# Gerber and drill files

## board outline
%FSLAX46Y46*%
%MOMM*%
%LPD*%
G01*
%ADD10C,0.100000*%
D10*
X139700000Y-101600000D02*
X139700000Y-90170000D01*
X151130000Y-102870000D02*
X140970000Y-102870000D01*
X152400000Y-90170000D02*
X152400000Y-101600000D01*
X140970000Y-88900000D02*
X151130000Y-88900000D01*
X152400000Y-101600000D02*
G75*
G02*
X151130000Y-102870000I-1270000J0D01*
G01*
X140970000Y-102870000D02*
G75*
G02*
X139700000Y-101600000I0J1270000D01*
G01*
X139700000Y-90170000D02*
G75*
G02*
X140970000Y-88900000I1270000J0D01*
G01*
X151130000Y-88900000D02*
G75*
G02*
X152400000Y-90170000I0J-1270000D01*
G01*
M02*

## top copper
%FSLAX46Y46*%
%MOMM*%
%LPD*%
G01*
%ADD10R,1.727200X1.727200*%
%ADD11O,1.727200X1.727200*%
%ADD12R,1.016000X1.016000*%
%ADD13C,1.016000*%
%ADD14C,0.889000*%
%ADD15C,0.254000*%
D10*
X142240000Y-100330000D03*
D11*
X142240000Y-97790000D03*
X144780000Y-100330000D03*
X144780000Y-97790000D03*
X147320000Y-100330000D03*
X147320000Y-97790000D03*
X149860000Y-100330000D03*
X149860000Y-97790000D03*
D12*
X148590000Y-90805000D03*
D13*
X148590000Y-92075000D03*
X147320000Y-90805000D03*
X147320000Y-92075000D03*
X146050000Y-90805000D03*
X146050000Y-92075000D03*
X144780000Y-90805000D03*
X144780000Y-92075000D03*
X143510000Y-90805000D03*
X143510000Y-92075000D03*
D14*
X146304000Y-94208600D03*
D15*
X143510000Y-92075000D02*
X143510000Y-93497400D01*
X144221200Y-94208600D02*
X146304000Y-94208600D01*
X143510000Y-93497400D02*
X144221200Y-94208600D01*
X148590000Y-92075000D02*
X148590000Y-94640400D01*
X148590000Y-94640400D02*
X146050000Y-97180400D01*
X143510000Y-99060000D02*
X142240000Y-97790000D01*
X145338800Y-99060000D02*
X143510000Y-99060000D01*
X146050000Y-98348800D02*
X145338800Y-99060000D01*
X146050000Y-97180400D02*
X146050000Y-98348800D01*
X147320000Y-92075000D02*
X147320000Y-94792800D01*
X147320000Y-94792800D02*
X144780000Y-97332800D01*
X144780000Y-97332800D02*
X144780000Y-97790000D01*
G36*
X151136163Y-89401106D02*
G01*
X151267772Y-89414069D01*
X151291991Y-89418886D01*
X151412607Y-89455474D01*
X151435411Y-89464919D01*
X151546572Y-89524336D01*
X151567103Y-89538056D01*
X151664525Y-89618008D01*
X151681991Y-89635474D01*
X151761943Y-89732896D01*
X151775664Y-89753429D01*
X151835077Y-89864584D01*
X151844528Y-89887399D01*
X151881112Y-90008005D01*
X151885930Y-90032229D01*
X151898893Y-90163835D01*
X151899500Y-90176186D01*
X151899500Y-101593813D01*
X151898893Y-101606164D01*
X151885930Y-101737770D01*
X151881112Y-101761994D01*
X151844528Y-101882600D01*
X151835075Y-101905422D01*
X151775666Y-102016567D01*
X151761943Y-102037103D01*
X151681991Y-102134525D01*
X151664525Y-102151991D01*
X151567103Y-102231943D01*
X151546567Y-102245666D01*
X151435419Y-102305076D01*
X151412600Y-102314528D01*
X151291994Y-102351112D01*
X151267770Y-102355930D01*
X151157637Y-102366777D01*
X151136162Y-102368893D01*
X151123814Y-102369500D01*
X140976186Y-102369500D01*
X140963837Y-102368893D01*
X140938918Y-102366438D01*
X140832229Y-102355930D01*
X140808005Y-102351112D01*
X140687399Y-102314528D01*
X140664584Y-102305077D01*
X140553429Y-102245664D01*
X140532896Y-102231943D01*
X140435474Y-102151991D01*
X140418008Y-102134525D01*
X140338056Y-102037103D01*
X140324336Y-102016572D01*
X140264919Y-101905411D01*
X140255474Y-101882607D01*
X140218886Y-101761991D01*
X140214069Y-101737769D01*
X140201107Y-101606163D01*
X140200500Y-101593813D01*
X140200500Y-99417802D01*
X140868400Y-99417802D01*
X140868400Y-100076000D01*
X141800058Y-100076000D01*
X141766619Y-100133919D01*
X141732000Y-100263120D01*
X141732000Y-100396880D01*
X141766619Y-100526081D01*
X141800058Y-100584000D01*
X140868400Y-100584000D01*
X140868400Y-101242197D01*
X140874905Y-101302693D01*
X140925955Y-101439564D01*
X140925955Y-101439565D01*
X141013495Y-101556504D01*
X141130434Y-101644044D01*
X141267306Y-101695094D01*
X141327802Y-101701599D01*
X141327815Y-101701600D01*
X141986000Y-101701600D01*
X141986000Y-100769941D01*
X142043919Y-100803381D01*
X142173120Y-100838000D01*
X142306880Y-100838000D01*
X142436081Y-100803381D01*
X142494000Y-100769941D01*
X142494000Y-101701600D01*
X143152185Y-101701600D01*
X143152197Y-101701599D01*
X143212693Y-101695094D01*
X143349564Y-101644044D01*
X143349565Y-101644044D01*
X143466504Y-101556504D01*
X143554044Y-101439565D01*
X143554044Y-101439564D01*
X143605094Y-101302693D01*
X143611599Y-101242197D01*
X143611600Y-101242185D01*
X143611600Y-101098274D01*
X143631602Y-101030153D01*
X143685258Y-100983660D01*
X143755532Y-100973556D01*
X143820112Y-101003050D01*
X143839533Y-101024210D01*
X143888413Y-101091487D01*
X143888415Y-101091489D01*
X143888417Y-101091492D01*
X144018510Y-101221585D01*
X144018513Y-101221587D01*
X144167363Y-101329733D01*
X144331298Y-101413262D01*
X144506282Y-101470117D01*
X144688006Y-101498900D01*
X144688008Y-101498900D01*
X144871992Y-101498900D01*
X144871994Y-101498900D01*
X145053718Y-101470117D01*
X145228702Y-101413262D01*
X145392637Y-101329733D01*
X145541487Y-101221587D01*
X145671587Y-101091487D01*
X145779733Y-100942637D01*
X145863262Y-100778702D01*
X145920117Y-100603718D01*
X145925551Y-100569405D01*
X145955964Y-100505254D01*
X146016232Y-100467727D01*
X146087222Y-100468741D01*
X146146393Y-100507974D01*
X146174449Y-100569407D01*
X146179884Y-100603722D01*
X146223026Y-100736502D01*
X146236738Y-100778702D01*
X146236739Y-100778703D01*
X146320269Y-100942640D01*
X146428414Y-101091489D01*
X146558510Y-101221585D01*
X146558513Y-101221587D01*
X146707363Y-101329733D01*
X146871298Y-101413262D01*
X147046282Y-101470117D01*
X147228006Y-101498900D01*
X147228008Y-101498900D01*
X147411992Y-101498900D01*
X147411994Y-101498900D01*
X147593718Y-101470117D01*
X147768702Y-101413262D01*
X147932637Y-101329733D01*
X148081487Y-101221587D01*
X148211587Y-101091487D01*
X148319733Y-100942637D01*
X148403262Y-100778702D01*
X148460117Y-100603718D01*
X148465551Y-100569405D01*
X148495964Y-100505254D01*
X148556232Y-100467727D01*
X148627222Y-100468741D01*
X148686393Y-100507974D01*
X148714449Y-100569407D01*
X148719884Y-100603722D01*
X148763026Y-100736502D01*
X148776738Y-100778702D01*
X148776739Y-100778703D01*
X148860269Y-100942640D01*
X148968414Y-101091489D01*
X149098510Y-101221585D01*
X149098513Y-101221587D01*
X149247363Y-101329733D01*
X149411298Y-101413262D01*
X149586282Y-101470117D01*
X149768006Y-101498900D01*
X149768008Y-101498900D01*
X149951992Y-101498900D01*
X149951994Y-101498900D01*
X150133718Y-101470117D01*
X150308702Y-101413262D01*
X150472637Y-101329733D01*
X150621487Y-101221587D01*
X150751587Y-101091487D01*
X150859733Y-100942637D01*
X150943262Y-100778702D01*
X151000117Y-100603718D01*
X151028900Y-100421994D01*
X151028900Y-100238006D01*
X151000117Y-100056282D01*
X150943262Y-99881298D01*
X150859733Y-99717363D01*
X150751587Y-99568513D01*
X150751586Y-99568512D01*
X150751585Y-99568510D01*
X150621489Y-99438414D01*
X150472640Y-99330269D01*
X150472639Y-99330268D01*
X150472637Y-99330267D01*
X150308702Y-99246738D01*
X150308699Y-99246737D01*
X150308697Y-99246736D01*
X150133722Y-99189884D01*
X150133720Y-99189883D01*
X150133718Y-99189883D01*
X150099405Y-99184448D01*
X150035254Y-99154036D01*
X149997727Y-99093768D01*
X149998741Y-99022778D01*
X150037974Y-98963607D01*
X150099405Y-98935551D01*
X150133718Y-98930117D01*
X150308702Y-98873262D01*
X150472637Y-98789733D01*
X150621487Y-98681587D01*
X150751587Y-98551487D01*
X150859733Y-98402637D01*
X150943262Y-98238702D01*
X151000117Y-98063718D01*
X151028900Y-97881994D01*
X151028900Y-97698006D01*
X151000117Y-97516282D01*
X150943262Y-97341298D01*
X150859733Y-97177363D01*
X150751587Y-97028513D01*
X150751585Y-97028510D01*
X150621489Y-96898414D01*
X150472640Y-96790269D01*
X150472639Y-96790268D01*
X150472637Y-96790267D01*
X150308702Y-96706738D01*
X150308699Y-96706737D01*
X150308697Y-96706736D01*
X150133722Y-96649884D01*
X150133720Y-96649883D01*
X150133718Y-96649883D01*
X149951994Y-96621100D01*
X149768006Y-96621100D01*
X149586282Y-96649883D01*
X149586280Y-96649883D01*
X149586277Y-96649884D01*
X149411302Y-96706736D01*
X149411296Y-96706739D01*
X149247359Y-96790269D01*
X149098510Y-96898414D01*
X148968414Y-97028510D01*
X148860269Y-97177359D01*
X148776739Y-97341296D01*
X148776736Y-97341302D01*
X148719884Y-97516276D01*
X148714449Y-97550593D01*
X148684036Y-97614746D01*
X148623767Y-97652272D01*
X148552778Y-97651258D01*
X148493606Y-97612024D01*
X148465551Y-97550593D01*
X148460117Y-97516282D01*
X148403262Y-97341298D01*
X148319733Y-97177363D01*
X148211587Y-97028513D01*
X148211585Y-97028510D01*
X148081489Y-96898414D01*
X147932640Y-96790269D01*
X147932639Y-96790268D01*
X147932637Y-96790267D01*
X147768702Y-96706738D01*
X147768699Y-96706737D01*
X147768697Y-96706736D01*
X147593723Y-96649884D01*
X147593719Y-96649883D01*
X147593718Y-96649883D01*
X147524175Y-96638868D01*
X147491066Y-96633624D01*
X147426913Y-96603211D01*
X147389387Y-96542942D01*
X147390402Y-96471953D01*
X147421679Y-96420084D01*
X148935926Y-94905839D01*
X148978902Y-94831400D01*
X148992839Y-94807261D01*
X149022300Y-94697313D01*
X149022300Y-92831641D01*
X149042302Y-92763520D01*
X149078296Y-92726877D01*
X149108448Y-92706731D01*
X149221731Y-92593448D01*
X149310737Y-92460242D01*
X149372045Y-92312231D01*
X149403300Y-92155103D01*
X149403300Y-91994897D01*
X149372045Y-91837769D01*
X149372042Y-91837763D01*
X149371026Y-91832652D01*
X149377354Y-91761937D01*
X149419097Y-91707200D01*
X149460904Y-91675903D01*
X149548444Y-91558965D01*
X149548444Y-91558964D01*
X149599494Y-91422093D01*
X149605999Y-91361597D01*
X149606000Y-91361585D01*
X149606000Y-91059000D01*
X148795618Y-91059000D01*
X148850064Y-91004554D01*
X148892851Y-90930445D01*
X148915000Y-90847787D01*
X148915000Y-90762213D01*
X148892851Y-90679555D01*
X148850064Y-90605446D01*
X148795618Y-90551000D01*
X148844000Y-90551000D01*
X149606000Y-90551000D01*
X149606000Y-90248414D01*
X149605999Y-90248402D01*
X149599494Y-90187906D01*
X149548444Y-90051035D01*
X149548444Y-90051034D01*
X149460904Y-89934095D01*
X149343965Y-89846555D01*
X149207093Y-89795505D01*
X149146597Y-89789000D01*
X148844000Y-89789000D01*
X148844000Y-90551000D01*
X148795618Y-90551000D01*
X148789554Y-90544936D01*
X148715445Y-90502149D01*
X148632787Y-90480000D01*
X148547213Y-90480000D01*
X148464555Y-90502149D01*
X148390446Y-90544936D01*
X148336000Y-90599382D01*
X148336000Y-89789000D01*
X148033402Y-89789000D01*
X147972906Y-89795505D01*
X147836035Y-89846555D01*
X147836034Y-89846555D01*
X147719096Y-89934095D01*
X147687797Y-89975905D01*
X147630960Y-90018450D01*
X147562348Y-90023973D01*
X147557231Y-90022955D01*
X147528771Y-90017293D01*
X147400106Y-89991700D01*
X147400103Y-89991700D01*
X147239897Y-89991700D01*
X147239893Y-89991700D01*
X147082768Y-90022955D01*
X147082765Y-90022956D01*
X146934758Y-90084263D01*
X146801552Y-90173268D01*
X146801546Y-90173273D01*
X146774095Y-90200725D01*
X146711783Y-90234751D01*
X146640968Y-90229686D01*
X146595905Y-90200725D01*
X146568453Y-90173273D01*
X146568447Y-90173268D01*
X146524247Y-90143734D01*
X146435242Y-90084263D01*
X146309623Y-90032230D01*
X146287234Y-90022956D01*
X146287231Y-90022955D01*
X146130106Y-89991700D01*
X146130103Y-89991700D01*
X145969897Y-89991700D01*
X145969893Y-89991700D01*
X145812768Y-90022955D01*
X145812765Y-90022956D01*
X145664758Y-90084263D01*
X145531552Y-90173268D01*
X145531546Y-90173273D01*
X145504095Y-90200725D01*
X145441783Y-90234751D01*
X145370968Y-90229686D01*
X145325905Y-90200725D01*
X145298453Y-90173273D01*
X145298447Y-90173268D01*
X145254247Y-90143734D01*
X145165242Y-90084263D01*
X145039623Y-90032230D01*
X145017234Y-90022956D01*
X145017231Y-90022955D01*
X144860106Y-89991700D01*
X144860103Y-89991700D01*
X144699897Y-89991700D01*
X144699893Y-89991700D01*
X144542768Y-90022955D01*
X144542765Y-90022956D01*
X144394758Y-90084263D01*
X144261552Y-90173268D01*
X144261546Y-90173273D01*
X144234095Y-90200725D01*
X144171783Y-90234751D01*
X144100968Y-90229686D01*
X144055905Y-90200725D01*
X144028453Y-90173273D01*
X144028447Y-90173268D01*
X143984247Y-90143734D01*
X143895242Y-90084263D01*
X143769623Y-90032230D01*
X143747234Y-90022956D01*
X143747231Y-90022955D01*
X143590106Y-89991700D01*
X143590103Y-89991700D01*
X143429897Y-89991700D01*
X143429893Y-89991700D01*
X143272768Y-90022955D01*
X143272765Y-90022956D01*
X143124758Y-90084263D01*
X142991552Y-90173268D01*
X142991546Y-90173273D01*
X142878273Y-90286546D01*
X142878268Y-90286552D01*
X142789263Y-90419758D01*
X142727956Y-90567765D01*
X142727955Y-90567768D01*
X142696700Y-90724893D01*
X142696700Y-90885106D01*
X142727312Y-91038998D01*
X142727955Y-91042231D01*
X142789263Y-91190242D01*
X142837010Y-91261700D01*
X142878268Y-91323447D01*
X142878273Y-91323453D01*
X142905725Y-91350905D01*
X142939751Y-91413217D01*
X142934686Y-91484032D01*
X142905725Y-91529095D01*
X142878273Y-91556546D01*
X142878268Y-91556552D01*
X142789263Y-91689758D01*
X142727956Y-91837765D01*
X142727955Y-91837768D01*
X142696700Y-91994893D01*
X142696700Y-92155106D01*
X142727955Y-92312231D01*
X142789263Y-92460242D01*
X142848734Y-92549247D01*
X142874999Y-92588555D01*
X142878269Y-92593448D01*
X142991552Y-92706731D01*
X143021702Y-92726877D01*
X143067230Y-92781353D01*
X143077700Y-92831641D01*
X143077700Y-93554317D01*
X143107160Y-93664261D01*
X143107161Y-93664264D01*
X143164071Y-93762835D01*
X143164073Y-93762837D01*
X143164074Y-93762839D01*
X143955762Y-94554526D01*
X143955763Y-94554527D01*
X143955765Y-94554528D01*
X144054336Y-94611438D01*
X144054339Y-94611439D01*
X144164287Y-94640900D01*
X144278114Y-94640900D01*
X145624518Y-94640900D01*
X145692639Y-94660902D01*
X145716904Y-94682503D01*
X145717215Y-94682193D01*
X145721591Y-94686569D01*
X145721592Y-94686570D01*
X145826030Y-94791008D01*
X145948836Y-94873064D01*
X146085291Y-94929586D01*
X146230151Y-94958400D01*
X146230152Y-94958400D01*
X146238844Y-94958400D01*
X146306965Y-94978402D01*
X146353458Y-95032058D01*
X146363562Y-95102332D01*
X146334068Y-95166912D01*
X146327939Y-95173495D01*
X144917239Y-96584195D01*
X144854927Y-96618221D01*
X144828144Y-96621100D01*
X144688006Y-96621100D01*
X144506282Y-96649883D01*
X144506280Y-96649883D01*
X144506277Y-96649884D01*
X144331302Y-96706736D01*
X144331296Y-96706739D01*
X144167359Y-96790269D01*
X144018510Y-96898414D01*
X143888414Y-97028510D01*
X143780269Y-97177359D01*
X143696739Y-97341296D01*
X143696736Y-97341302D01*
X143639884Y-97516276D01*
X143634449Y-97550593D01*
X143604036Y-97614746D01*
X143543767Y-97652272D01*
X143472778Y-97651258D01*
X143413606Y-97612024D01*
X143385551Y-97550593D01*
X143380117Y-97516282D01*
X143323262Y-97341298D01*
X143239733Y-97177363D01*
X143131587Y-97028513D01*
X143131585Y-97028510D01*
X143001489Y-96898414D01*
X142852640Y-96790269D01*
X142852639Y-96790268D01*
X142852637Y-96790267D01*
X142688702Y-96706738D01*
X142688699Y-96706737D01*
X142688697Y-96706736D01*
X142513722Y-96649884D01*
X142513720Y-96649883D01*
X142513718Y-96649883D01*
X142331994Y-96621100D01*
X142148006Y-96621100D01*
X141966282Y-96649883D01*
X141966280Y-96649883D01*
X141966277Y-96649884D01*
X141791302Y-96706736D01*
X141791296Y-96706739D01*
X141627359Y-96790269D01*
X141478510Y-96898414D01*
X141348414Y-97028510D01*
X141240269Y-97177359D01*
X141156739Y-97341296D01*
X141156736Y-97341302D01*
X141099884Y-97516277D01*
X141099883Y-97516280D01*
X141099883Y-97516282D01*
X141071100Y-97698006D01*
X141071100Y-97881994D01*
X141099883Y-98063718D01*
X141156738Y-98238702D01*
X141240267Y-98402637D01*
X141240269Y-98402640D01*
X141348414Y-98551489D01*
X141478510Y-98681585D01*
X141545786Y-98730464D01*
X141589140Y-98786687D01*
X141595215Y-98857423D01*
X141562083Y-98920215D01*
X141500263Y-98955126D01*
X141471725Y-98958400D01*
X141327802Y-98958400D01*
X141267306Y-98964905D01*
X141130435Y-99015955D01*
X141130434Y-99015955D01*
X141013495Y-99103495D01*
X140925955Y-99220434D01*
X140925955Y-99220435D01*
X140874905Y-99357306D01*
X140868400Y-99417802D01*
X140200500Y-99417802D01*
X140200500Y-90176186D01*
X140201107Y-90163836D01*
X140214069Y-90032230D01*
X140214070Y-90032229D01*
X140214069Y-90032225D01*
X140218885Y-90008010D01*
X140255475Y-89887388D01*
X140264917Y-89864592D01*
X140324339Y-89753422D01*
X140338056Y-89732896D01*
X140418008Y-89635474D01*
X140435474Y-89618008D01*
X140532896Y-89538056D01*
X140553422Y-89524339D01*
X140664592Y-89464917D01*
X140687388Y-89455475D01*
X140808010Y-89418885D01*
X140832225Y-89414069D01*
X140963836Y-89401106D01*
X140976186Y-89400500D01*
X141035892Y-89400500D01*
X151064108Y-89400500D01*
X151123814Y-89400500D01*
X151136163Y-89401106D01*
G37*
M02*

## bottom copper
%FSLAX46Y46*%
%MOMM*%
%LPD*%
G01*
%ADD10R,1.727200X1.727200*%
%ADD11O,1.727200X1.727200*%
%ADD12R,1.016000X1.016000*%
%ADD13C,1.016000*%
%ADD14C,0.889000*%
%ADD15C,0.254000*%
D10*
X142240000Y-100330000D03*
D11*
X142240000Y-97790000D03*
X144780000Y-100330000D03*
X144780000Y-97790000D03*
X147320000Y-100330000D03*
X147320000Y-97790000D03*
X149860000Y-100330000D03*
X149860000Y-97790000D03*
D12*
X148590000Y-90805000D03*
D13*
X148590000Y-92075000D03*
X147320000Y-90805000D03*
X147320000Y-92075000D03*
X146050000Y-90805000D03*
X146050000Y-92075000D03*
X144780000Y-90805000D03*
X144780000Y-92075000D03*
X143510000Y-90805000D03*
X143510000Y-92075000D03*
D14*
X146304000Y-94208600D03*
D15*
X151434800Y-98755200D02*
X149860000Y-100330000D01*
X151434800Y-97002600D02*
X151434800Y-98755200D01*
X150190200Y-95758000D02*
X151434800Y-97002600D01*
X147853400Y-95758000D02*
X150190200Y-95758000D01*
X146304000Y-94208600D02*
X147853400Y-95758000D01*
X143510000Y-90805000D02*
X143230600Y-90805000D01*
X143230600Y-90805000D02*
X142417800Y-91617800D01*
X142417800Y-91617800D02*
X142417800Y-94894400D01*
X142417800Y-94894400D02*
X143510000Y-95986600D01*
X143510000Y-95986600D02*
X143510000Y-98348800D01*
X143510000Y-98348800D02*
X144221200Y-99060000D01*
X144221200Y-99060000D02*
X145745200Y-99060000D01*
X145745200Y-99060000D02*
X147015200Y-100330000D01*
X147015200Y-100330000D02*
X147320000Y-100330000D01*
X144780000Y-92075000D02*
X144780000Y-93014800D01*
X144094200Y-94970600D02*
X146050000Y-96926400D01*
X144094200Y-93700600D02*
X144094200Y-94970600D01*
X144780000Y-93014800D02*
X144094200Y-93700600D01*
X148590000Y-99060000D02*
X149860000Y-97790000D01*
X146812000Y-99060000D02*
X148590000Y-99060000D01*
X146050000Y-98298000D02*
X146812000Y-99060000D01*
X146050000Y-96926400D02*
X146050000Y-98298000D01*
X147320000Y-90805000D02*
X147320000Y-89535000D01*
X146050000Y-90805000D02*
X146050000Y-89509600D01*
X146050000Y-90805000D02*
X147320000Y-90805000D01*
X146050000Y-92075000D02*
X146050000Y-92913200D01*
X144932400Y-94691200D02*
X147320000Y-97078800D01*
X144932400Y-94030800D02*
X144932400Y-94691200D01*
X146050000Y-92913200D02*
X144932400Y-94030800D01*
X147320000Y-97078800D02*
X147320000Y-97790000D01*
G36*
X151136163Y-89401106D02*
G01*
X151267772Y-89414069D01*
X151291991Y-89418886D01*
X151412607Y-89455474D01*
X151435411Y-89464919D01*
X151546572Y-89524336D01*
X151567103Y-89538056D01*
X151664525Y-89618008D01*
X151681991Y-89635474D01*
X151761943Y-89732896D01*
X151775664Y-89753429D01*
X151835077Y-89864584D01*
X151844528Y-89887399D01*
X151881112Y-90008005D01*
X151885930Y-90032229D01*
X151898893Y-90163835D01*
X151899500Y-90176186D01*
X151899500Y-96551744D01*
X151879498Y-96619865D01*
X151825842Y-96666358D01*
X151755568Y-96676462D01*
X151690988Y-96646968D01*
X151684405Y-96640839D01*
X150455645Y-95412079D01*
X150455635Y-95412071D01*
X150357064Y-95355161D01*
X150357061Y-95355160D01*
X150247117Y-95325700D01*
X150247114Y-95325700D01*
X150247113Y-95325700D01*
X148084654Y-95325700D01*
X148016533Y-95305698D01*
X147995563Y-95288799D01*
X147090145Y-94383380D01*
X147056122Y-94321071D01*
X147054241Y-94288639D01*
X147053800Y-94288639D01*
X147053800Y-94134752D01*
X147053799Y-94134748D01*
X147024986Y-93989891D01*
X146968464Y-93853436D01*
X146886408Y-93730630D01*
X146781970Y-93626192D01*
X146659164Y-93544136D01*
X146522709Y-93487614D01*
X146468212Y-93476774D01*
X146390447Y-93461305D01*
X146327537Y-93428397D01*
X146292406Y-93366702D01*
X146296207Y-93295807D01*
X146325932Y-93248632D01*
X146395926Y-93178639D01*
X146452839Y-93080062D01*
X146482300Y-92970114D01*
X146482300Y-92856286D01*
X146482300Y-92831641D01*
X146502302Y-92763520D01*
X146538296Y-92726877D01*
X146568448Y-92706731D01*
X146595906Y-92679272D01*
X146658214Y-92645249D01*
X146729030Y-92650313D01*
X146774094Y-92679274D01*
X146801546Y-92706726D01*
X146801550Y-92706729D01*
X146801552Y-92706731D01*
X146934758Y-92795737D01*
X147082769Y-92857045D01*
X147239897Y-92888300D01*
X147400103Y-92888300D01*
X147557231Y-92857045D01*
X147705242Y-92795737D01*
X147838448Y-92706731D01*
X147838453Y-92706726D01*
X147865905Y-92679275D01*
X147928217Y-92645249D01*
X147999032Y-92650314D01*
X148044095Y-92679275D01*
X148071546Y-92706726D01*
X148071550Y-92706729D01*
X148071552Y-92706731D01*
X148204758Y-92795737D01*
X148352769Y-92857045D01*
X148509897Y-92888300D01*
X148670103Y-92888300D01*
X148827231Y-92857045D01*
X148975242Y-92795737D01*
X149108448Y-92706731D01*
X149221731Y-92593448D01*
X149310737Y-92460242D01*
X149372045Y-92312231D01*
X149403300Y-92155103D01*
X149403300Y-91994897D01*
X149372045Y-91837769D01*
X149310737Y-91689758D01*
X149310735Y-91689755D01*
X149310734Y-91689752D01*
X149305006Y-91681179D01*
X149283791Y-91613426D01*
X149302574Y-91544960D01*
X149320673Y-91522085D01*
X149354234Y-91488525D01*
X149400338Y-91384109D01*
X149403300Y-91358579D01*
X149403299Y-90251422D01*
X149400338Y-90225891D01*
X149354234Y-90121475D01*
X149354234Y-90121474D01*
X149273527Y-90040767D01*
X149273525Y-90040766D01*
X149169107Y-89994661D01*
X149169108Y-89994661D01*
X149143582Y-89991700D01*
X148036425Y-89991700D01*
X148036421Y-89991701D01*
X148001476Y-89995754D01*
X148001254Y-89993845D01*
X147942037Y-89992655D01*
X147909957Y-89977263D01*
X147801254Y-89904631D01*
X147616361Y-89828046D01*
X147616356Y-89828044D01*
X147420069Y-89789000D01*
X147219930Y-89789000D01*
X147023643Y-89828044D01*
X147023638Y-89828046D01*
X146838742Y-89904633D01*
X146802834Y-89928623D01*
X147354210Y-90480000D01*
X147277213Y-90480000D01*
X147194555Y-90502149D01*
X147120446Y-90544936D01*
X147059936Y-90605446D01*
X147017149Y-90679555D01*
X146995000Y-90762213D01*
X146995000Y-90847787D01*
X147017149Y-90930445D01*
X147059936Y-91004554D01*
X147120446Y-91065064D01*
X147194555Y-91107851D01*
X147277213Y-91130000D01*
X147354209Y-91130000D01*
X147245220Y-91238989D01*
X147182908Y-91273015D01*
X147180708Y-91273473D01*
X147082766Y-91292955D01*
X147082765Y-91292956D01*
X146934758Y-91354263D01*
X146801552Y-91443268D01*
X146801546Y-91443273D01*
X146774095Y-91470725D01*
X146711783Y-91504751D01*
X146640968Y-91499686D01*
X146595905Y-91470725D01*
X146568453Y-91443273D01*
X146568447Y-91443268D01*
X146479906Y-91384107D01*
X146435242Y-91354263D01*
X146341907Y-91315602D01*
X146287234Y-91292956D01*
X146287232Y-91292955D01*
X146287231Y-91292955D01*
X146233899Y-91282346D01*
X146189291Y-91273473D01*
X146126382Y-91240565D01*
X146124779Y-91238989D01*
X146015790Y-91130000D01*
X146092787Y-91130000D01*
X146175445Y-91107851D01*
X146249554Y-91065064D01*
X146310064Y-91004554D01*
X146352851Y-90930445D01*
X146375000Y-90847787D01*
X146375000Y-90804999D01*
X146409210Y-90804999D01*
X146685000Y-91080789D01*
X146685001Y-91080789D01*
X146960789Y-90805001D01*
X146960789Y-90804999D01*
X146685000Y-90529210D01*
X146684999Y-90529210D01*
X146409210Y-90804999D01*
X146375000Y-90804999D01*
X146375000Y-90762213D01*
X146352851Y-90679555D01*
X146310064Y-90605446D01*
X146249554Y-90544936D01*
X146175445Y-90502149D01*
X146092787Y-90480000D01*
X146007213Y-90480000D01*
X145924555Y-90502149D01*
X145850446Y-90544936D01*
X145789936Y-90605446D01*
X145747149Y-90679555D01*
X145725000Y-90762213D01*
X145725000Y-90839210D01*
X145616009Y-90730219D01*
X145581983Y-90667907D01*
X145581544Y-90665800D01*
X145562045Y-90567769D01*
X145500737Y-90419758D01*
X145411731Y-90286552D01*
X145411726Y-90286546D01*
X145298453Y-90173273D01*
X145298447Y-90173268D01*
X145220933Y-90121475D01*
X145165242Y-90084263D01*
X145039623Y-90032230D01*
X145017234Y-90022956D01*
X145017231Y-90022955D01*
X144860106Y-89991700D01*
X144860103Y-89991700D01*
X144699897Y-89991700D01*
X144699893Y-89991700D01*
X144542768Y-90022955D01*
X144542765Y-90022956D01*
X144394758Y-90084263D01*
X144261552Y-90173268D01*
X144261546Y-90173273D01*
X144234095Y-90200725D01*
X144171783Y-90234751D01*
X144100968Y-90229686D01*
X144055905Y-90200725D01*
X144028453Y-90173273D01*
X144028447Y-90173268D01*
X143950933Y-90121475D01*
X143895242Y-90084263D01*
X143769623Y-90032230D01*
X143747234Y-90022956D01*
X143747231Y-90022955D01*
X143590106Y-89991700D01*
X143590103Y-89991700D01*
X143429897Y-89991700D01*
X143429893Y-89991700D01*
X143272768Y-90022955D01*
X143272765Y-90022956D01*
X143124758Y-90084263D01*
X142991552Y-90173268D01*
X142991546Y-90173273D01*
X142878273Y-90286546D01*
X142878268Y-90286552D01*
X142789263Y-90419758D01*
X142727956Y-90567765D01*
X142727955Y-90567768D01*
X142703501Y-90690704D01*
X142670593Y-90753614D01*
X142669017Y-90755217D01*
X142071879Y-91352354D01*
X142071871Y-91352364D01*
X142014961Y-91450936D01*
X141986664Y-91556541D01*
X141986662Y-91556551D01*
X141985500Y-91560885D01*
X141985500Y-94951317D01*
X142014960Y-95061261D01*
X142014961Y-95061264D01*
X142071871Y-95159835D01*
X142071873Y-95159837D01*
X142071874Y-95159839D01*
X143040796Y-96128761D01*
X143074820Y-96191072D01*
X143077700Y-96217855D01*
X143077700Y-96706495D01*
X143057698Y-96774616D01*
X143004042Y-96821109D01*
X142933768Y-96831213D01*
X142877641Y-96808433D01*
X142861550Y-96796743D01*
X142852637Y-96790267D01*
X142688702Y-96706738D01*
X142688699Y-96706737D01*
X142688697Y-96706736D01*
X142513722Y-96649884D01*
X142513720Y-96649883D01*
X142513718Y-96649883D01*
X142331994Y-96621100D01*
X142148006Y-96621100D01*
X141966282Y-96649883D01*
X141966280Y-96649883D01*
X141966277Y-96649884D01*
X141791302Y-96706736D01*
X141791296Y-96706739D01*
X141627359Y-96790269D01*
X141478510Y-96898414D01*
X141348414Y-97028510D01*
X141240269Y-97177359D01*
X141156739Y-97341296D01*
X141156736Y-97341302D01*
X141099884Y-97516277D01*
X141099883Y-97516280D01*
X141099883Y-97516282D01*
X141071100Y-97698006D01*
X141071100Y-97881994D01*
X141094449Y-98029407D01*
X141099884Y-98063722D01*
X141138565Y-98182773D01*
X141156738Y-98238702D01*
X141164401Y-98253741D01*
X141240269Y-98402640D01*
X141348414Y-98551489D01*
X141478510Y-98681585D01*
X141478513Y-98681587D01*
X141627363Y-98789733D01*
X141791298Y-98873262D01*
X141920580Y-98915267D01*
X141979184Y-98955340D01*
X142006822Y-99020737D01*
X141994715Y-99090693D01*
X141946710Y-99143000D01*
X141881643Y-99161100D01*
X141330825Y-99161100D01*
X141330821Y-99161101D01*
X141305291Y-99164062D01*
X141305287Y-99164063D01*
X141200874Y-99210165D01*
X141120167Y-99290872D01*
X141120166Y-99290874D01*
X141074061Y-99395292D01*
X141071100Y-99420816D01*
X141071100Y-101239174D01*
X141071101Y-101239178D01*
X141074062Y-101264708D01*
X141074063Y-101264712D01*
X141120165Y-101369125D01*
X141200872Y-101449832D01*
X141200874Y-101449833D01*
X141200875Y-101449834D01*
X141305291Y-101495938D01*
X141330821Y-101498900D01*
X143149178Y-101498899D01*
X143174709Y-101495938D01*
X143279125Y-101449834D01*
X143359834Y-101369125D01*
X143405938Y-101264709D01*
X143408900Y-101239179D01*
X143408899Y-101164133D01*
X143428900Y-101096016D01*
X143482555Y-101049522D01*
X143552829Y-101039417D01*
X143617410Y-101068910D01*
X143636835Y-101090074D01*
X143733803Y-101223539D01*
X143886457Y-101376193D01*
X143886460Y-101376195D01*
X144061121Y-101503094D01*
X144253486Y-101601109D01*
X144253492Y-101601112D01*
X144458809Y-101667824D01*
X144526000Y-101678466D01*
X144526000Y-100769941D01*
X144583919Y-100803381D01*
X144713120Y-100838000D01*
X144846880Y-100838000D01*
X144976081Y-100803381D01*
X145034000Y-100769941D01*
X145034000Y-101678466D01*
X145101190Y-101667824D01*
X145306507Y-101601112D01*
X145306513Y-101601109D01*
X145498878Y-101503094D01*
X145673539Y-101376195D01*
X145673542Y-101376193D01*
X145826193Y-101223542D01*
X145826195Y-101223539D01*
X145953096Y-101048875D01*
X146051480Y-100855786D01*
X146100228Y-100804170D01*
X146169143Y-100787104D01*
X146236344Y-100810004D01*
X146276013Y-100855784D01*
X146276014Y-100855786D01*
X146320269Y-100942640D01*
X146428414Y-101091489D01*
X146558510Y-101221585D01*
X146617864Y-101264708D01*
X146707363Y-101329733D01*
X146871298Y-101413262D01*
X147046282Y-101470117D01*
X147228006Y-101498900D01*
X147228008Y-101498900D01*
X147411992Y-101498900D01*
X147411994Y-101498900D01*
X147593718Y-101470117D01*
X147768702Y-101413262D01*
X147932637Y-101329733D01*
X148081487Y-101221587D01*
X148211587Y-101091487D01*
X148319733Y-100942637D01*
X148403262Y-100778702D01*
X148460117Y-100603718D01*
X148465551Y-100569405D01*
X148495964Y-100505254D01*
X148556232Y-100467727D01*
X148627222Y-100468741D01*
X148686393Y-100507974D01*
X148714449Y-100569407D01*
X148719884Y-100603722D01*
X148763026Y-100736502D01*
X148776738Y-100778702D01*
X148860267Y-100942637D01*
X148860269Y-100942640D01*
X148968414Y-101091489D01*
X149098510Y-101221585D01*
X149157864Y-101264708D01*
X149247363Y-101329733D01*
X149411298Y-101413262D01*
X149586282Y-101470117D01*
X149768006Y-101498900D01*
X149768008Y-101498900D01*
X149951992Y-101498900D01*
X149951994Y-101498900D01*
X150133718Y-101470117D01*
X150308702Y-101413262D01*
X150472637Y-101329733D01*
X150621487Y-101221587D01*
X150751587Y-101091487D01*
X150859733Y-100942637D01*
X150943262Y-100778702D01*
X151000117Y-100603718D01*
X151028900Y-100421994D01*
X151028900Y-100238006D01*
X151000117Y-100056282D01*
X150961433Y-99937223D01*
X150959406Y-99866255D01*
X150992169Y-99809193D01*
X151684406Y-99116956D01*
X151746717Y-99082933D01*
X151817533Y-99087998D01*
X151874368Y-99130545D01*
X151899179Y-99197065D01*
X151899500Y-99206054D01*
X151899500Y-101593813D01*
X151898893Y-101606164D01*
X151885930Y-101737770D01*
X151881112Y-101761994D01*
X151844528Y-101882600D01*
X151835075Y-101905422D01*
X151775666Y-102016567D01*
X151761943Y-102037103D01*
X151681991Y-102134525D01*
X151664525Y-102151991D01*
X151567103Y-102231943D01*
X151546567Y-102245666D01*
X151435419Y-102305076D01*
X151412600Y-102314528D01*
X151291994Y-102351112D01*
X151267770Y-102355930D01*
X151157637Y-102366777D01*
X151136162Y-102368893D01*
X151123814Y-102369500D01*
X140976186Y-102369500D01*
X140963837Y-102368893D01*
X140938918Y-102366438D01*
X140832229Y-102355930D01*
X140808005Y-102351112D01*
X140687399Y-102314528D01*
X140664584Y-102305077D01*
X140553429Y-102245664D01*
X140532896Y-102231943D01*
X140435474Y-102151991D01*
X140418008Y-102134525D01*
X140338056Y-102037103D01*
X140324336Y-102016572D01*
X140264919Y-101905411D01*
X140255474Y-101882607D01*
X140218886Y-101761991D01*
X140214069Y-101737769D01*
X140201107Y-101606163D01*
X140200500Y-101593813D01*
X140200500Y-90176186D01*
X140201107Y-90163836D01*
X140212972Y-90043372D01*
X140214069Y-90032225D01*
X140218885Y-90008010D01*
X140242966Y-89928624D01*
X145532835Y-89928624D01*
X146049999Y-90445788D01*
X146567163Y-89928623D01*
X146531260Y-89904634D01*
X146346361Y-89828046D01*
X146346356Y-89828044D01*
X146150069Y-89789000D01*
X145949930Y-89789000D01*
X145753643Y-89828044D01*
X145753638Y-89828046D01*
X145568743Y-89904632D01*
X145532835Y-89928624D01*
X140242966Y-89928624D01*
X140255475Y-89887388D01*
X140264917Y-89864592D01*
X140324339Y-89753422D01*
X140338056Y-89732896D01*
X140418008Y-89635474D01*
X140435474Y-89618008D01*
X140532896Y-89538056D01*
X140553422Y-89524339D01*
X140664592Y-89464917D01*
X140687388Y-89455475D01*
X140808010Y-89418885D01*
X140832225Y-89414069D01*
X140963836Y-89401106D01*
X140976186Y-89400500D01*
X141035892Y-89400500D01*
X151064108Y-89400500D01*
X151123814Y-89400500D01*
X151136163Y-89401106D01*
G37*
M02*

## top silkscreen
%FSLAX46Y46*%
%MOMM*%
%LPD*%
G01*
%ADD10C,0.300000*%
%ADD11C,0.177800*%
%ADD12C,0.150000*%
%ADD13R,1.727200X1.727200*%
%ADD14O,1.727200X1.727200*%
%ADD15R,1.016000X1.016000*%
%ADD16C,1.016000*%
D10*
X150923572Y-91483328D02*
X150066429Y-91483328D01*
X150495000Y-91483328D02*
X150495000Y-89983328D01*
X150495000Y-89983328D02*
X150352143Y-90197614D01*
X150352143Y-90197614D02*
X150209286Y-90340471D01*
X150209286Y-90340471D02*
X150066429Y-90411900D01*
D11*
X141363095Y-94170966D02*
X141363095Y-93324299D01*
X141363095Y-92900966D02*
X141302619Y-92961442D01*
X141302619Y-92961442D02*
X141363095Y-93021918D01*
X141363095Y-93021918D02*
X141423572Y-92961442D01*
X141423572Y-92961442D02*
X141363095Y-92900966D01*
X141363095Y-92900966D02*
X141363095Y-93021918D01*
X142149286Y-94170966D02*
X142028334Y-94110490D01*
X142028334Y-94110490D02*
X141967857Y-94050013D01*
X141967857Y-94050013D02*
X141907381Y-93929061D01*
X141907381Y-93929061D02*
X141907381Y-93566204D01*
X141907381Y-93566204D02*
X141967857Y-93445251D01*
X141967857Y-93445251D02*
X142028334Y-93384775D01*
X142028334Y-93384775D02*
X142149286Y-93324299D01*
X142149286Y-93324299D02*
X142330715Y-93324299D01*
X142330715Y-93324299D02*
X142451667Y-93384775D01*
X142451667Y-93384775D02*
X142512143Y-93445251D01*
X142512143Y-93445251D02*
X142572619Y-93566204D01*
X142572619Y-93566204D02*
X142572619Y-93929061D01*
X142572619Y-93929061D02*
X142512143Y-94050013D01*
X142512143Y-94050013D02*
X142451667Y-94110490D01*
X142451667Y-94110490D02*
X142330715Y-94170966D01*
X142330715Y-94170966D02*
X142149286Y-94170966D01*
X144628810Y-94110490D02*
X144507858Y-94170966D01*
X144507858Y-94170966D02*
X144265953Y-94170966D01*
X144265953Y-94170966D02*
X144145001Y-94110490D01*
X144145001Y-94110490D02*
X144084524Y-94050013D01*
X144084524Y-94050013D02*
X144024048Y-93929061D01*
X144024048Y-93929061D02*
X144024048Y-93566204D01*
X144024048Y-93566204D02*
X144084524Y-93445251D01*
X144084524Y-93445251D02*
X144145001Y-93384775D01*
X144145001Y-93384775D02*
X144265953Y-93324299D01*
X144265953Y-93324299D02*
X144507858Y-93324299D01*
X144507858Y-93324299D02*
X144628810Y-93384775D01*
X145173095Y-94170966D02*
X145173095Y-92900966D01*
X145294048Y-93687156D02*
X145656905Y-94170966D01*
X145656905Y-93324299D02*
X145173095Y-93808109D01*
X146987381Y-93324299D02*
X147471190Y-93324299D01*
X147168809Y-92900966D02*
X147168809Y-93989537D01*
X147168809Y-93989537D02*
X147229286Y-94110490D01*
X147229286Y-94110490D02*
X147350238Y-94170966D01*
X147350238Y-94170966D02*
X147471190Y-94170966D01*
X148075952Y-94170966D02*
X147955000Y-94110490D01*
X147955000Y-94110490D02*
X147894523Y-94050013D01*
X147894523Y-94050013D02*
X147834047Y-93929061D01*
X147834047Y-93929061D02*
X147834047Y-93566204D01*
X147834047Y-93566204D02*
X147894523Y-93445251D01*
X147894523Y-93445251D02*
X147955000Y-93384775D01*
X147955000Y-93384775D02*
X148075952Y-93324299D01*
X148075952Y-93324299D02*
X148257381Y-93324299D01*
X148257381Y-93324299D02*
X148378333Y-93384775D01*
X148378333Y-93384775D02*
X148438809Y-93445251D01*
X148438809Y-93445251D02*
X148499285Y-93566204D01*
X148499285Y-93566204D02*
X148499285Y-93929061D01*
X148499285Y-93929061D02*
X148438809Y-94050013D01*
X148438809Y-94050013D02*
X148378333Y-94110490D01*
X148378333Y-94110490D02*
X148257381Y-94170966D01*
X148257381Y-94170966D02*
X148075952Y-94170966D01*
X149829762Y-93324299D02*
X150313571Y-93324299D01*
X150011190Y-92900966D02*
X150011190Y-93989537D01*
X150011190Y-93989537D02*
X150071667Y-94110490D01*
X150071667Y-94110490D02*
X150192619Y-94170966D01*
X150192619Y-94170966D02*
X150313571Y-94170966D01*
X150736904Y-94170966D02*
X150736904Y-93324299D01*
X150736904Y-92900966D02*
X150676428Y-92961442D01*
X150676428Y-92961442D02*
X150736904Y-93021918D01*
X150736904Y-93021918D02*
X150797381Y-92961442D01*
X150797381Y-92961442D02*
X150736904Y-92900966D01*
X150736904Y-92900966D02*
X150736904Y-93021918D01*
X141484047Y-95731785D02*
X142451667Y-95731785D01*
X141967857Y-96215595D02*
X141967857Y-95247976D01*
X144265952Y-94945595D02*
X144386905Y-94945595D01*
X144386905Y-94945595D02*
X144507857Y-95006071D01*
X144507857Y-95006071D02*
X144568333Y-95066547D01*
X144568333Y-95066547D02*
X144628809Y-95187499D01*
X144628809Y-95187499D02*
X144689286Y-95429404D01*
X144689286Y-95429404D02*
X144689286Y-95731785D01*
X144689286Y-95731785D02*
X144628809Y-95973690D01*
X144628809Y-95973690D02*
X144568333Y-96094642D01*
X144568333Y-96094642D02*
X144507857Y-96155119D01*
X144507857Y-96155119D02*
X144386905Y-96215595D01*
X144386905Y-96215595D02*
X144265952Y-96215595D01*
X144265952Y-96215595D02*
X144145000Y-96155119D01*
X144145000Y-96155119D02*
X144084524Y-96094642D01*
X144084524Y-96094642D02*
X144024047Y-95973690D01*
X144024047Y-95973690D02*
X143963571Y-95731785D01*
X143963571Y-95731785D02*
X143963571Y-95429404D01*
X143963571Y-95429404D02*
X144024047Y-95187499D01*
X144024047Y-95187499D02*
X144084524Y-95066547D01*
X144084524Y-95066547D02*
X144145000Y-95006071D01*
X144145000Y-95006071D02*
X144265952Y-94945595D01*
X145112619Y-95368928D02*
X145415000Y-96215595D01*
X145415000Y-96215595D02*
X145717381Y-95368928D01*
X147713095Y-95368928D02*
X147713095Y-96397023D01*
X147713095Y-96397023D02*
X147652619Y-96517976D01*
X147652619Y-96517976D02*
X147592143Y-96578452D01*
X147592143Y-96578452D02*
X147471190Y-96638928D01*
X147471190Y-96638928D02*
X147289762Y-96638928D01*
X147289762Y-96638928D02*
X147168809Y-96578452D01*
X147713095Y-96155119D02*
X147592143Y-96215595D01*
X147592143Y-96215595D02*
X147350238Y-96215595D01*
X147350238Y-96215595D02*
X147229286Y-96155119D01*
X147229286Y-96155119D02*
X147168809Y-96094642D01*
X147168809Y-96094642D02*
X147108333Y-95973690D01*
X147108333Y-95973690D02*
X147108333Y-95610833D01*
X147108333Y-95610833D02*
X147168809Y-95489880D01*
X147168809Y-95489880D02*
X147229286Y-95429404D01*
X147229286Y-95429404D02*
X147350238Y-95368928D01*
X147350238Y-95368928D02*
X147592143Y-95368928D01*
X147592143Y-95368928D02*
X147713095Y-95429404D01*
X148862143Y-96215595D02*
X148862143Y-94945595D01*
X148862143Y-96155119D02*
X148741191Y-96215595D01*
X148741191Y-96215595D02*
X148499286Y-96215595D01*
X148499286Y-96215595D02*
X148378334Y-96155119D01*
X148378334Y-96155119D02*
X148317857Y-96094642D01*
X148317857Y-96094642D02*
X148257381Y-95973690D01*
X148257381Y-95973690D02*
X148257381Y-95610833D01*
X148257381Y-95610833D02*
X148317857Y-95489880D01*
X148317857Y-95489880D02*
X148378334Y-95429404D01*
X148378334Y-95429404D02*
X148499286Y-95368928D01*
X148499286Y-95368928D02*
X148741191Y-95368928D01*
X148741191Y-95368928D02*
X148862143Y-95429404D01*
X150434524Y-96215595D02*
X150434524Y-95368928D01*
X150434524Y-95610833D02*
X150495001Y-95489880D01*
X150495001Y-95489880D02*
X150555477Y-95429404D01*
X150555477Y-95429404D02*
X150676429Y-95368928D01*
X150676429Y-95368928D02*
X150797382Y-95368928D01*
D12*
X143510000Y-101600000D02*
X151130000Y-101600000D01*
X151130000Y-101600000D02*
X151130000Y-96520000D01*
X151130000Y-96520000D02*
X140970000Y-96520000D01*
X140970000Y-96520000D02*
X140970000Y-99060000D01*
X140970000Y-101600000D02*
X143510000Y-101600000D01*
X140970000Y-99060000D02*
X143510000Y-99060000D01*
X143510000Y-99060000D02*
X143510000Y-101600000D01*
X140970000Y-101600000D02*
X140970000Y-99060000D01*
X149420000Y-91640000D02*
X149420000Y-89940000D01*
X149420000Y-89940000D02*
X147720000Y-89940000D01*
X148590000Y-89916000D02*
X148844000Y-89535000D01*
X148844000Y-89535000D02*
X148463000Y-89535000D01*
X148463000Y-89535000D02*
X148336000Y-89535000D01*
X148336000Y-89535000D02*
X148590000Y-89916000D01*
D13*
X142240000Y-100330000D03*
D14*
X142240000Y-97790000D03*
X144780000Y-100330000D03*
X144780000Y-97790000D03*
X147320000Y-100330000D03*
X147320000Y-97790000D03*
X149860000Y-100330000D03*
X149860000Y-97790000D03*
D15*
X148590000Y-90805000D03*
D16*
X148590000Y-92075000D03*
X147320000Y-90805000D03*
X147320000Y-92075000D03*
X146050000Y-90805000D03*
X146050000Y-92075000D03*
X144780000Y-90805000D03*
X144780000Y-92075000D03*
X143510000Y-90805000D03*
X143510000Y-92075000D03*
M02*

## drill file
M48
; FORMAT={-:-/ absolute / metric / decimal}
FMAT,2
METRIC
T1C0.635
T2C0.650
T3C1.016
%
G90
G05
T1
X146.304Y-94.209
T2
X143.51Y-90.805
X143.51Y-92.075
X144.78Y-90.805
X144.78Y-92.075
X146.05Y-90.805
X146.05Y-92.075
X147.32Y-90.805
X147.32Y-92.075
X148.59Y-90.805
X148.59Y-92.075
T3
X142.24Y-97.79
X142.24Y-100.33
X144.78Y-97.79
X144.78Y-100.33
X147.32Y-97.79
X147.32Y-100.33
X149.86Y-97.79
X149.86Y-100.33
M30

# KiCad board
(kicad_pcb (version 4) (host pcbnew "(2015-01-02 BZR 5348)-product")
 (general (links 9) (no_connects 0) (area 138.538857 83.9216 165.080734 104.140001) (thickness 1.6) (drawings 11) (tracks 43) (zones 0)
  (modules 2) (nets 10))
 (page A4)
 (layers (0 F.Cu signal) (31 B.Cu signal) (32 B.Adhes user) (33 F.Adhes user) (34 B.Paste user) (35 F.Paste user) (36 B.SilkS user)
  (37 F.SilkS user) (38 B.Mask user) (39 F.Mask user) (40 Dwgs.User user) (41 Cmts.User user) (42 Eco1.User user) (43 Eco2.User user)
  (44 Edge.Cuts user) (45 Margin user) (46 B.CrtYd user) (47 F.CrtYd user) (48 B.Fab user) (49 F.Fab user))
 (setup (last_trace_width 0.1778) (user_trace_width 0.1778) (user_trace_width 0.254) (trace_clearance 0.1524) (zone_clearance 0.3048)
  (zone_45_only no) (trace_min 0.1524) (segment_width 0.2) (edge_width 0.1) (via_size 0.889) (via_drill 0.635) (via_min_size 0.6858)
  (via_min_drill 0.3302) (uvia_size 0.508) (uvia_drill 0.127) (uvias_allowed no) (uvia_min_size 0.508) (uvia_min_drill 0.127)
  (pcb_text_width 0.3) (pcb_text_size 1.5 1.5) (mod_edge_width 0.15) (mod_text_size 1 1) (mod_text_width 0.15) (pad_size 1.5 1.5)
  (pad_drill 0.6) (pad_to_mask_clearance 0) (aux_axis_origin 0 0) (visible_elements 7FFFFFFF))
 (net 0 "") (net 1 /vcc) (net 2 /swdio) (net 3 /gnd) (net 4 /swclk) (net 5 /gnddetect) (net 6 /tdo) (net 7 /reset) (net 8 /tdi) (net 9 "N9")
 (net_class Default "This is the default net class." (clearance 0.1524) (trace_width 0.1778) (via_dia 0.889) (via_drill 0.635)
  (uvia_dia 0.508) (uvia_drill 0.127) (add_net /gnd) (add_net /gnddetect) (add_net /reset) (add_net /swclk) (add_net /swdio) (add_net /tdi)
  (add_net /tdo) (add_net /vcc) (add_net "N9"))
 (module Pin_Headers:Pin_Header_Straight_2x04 (layer F.Cu) (at 146.05 99.06)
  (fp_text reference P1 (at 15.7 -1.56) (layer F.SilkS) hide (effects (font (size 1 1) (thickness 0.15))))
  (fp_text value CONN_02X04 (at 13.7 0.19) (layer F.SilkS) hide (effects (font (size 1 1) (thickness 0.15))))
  (fp_line (start -2.54 2.54) (end 5.08 2.54) (layer F.SilkS) (width 0.15))
  (fp_line (start 5.08 2.54) (end 5.08 -2.54) (layer F.SilkS) (width 0.15))
  (fp_line (start 5.08 -2.54) (end -5.08 -2.54) (layer F.SilkS) (width 0.15))
  (fp_line (start -5.08 -2.54) (end -5.08 0) (layer F.SilkS) (width 0.15))
  (fp_line (start -5.08 2.54) (end -2.54 2.54) (layer F.SilkS) (width 0.15))
  (fp_line (start -5.08 0) (end -2.54 0) (layer F.SilkS) (width 0.15))
  (fp_line (start -2.54 0) (end -2.54 2.54) (layer F.SilkS) (width 0.15))
  (fp_line (start -5.08 2.54) (end -5.08 0) (layer F.SilkS) (width 0.15))
  (pad 1 thru_hole rect (at -3.81 1.27) (size 1.7272 1.7272) (drill 1.016) (layers *.Cu *.Mask F.SilkS) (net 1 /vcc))
  (pad 2 thru_hole oval (at -3.81 -1.27) (size 1.7272 1.7272) (drill 1.016) (layers *.Cu *.Mask F.SilkS) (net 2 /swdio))
  (pad 3 thru_hole oval (at -1.27 1.27) (size 1.7272 1.7272) (drill 1.016) (layers *.Cu *.Mask F.SilkS) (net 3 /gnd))
  (pad 4 thru_hole oval (at -1.27 -1.27) (size 1.7272 1.7272) (drill 1.016) (layers *.Cu *.Mask F.SilkS) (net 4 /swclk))
  (pad 5 thru_hole oval (at 1.27 1.27) (size 1.7272 1.7272) (drill 1.016) (layers *.Cu *.Mask F.SilkS) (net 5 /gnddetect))
  (pad 6 thru_hole oval (at 1.27 -1.27) (size 1.7272 1.7272) (drill 1.016) (layers *.Cu *.Mask F.SilkS) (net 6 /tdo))
  (pad 7 thru_hole oval (at 3.81 1.27) (size 1.7272 1.7272) (drill 1.016) (layers *.Cu *.Mask F.SilkS) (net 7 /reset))
  (pad 8 thru_hole oval (at 3.81 -1.27) (size 1.7272 1.7272) (drill 1.016) (layers *.Cu *.Mask F.SilkS) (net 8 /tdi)))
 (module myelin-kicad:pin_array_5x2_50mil (layer F.Cu) (at 147.32 91.44 180)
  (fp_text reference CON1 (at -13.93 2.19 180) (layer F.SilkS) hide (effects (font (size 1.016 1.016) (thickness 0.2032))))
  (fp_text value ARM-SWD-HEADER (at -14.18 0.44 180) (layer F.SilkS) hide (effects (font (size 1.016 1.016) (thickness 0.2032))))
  (fp_line (start -2.1 -0.2) (end -2.1 1.5) (layer F.SilkS) (width 0.15))
  (fp_line (start -2.1 1.5) (end -0.4 1.5) (layer F.SilkS) (width 0.15))
  (fp_line (start -1.27 1.524) (end -1.524 1.905) (layer F.SilkS) (width 0.15))
  (fp_line (start -1.524 1.905) (end -1.143 1.905) (layer F.SilkS) (width 0.15))
  (fp_line (start -1.143 1.905) (end -1.016 1.905) (layer F.SilkS) (width 0.15))
  (fp_line (start -1.016 1.905) (end -1.27 1.524) (layer F.SilkS) (width 0.15))
  (pad 1 thru_hole rect (at -1.27 0.635 180) (size 1.016 1.016) (drill 0.65) (layers *.Cu *.Mask F.SilkS) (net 1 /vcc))
  (pad 2 thru_hole circle (at -1.27 -0.635 180) (size 1.016 1.016) (drill 0.65) (layers *.Cu *.Mask F.SilkS) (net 2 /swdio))
  (pad 3 thru_hole circle (at 0 0.635 180) (size 1.016 1.016) (drill 0.65) (layers *.Cu *.Mask F.SilkS) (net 3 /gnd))
  (pad 4 thru_hole circle (at 0 -0.635 180) (size 1.016 1.016) (drill 0.65) (layers *.Cu *.Mask F.SilkS) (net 4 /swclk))
  (pad 5 thru_hole circle (at 1.27 0.635 180) (size 1.016 1.016) (drill 0.65) (layers *.Cu *.Mask F.SilkS) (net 3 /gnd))
  (pad 6 thru_hole circle (at 1.27 -0.635 180) (size 1.016 1.016) (drill 0.65) (layers *.Cu *.Mask F.SilkS) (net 6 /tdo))
  (pad 7 thru_hole circle (at 2.54 0.635 180) (size 1.016 1.016) (drill 0.65) (layers *.Cu *.Mask F.SilkS) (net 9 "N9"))
  (pad 8 thru_hole circle (at 2.54 -0.635 180) (size 1.016 1.016) (drill 0.65) (layers *.Cu *.Mask F.SilkS) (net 8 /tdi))
  (pad 9 thru_hole circle (at 3.81 0.635 180) (size 1.016 1.016) (drill 0.65) (layers *.Cu *.Mask F.SilkS) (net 5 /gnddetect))
  (pad 10 thru_hole circle (at 3.81 -0.635 180) (size 1.016 1.016) (drill 0.65) (layers *.Cu *.Mask F.SilkS) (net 7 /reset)))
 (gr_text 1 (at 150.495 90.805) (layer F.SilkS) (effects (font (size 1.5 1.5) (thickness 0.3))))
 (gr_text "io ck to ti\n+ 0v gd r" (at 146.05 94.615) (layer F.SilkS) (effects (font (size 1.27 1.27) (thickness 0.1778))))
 (gr_line (start 139.7 101.6) (end 139.7 90.17) (angle 90) (layer Edge.Cuts) (width 0.1))
 (gr_line (start 151.13 102.87) (end 140.97 102.87) (angle 90) (layer Edge.Cuts) (width 0.1))
 (gr_line (start 152.4 90.17) (end 152.4 101.6) (angle 90) (layer Edge.Cuts) (width 0.1))
 (gr_line (start 140.97 88.9) (end 151.13 88.9) (angle 90) (layer Edge.Cuts) (width 0.1))
 (gr_arc (start 151.13 101.6) (end 152.4 101.6) (angle 90) (layer Edge.Cuts) (width 0.1))
 (gr_arc (start 140.97 101.6) (end 140.97 102.87) (angle 90) (layer Edge.Cuts) (width 0.1))
 (gr_arc (start 140.97 90.17) (end 139.7 90.17) (angle 90) (layer Edge.Cuts) (width 0.1))
 (gr_arc (start 151.13 90.17) (end 151.13 88.9) (angle 90) (layer Edge.Cuts) (width 0.1))
 (segment (start 143.51 92.075) (end 143.51 93.4974) (width 0.254) (layer F.Cu) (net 7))
 (segment (start 151.4348 98.7552) (end 149.86 100.33) (width 0.254) (layer B.Cu) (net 7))
 (segment (start 151.4348 97.0026) (end 151.4348 98.7552) (width 0.254) (layer B.Cu) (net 7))
 (segment (start 150.1902 95.758) (end 151.4348 97.0026) (width 0.254) (layer B.Cu) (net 7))
 (segment (start 147.8534 95.758) (end 150.1902 95.758) (width 0.254) (layer B.Cu) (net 7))
 (segment (start 146.304 94.2086) (end 147.8534 95.758) (width 0.254) (layer B.Cu) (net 7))
 (via (at 146.304 94.2086) (size 0.889) (layers F.Cu B.Cu) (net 7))
 (segment (start 144.2212 94.2086) (end 146.304 94.2086) (width 0.254) (layer F.Cu) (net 7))
 (segment (start 143.51 93.4974) (end 144.2212 94.2086) (width 0.254) (layer F.Cu) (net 7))
 (segment (start 143.51 90.805) (end 143.2306 90.805) (width 0.254) (layer B.Cu) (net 5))
 (segment (start 143.2306 90.805) (end 142.4178 91.6178) (width 0.254) (layer B.Cu) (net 5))
 (segment (start 142.4178 91.6178) (end 142.4178 94.8944) (width 0.254) (layer B.Cu) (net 5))
 (segment (start 142.4178 94.8944) (end 143.51 95.9866) (width 0.254) (layer B.Cu) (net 5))
 (segment (start 143.51 95.9866) (end 143.51 98.3488) (width 0.254) (layer B.Cu) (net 5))
 (segment (start 143.51 98.3488) (end 144.2212 99.06) (width 0.254) (layer B.Cu) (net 5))
 (segment (start 144.2212 99.06) (end 145.7452 99.06) (width 0.254) (layer B.Cu) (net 5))
 (segment (start 145.7452 99.06) (end 147.0152 100.33) (width 0.254) (layer B.Cu) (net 5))
 (segment (start 147.0152 100.33) (end 147.32 100.33) (width 0.254) (layer B.Cu) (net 5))
 (segment (start 144.78 92.075) (end 144.78 93.0148) (width 0.254) (layer B.Cu) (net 8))
 (segment (start 144.0942 94.9706) (end 146.05 96.9264) (width 0.254) (layer B.Cu) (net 8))
 (segment (start 144.0942 93.7006) (end 144.0942 94.9706) (width 0.254) (layer B.Cu) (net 8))
 (segment (start 144.78 93.0148) (end 144.0942 93.7006) (width 0.254) (layer B.Cu) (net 8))
 (segment (start 148.59 99.06) (end 149.86 97.79) (width 0.254) (layer B.Cu) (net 8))
 (segment (start 146.812 99.06) (end 148.59 99.06) (width 0.254) (layer B.Cu) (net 8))
 (segment (start 146.05 98.298) (end 146.812 99.06) (width 0.254) (layer B.Cu) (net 8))
 (segment (start 146.05 96.9264) (end 146.05 98.298) (width 0.254) (layer B.Cu) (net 8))
 (segment (start 148.59 92.075) (end 148.59 94.6404) (width 0.254) (layer F.Cu) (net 2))
 (segment (start 148.59 94.6404) (end 146.05 97.1804) (width 0.254) (layer F.Cu) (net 2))
 (segment (start 143.51 99.06) (end 142.24 97.79) (width 0.254) (layer F.Cu) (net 2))
 (segment (start 145.3388 99.06) (end 143.51 99.06) (width 0.254) (layer F.Cu) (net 2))
 (segment (start 146.05 98.3488) (end 145.3388 99.06) (width 0.254) (layer F.Cu) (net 2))
 (segment (start 146.05 97.1804) (end 146.05 98.3488) (width 0.254) (layer F.Cu) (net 2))
 (segment (start 147.32 90.805) (end 147.32 89.535) (width 0.254) (layer B.Cu) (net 3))
 (segment (start 146.05 90.805) (end 146.05 89.5096) (width 0.254) (layer B.Cu) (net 3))
 (segment (start 146.05 90.805) (end 147.32 90.805) (width 0.254) (layer B.Cu) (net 3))
 (segment (start 147.32 92.075) (end 147.32 94.7928) (width 0.254) (layer F.Cu) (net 4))
 (segment (start 147.32 94.7928) (end 144.78 97.3328) (width 0.254) (layer F.Cu) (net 4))
 (segment (start 144.78 97.3328) (end 144.78 97.79) (width 0.254) (layer F.Cu) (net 4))
 (segment (start 146.05 92.075) (end 146.05 92.9132) (width 0.254) (layer B.Cu) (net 6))
 (segment (start 144.9324 94.6912) (end 147.32 97.0788) (width 0.254) (layer B.Cu) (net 6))
 (segment (start 144.9324 94.0308) (end 144.9324 94.6912) (width 0.254) (layer B.Cu) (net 6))
 (segment (start 146.05 92.9132) (end 144.9324 94.0308) (width 0.254) (layer B.Cu) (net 6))
 (segment (start 147.32 97.0788) (end 147.32 97.79) (width 0.254) (layer B.Cu) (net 6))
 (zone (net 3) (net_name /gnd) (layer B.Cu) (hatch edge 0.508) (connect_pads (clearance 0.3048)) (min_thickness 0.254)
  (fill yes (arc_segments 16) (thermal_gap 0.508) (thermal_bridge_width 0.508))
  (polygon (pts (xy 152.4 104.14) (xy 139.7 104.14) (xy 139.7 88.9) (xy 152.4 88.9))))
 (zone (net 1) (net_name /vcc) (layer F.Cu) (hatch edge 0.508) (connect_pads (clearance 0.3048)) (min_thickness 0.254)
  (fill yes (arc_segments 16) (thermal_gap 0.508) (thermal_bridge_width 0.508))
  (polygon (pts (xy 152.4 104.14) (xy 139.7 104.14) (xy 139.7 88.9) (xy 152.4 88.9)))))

